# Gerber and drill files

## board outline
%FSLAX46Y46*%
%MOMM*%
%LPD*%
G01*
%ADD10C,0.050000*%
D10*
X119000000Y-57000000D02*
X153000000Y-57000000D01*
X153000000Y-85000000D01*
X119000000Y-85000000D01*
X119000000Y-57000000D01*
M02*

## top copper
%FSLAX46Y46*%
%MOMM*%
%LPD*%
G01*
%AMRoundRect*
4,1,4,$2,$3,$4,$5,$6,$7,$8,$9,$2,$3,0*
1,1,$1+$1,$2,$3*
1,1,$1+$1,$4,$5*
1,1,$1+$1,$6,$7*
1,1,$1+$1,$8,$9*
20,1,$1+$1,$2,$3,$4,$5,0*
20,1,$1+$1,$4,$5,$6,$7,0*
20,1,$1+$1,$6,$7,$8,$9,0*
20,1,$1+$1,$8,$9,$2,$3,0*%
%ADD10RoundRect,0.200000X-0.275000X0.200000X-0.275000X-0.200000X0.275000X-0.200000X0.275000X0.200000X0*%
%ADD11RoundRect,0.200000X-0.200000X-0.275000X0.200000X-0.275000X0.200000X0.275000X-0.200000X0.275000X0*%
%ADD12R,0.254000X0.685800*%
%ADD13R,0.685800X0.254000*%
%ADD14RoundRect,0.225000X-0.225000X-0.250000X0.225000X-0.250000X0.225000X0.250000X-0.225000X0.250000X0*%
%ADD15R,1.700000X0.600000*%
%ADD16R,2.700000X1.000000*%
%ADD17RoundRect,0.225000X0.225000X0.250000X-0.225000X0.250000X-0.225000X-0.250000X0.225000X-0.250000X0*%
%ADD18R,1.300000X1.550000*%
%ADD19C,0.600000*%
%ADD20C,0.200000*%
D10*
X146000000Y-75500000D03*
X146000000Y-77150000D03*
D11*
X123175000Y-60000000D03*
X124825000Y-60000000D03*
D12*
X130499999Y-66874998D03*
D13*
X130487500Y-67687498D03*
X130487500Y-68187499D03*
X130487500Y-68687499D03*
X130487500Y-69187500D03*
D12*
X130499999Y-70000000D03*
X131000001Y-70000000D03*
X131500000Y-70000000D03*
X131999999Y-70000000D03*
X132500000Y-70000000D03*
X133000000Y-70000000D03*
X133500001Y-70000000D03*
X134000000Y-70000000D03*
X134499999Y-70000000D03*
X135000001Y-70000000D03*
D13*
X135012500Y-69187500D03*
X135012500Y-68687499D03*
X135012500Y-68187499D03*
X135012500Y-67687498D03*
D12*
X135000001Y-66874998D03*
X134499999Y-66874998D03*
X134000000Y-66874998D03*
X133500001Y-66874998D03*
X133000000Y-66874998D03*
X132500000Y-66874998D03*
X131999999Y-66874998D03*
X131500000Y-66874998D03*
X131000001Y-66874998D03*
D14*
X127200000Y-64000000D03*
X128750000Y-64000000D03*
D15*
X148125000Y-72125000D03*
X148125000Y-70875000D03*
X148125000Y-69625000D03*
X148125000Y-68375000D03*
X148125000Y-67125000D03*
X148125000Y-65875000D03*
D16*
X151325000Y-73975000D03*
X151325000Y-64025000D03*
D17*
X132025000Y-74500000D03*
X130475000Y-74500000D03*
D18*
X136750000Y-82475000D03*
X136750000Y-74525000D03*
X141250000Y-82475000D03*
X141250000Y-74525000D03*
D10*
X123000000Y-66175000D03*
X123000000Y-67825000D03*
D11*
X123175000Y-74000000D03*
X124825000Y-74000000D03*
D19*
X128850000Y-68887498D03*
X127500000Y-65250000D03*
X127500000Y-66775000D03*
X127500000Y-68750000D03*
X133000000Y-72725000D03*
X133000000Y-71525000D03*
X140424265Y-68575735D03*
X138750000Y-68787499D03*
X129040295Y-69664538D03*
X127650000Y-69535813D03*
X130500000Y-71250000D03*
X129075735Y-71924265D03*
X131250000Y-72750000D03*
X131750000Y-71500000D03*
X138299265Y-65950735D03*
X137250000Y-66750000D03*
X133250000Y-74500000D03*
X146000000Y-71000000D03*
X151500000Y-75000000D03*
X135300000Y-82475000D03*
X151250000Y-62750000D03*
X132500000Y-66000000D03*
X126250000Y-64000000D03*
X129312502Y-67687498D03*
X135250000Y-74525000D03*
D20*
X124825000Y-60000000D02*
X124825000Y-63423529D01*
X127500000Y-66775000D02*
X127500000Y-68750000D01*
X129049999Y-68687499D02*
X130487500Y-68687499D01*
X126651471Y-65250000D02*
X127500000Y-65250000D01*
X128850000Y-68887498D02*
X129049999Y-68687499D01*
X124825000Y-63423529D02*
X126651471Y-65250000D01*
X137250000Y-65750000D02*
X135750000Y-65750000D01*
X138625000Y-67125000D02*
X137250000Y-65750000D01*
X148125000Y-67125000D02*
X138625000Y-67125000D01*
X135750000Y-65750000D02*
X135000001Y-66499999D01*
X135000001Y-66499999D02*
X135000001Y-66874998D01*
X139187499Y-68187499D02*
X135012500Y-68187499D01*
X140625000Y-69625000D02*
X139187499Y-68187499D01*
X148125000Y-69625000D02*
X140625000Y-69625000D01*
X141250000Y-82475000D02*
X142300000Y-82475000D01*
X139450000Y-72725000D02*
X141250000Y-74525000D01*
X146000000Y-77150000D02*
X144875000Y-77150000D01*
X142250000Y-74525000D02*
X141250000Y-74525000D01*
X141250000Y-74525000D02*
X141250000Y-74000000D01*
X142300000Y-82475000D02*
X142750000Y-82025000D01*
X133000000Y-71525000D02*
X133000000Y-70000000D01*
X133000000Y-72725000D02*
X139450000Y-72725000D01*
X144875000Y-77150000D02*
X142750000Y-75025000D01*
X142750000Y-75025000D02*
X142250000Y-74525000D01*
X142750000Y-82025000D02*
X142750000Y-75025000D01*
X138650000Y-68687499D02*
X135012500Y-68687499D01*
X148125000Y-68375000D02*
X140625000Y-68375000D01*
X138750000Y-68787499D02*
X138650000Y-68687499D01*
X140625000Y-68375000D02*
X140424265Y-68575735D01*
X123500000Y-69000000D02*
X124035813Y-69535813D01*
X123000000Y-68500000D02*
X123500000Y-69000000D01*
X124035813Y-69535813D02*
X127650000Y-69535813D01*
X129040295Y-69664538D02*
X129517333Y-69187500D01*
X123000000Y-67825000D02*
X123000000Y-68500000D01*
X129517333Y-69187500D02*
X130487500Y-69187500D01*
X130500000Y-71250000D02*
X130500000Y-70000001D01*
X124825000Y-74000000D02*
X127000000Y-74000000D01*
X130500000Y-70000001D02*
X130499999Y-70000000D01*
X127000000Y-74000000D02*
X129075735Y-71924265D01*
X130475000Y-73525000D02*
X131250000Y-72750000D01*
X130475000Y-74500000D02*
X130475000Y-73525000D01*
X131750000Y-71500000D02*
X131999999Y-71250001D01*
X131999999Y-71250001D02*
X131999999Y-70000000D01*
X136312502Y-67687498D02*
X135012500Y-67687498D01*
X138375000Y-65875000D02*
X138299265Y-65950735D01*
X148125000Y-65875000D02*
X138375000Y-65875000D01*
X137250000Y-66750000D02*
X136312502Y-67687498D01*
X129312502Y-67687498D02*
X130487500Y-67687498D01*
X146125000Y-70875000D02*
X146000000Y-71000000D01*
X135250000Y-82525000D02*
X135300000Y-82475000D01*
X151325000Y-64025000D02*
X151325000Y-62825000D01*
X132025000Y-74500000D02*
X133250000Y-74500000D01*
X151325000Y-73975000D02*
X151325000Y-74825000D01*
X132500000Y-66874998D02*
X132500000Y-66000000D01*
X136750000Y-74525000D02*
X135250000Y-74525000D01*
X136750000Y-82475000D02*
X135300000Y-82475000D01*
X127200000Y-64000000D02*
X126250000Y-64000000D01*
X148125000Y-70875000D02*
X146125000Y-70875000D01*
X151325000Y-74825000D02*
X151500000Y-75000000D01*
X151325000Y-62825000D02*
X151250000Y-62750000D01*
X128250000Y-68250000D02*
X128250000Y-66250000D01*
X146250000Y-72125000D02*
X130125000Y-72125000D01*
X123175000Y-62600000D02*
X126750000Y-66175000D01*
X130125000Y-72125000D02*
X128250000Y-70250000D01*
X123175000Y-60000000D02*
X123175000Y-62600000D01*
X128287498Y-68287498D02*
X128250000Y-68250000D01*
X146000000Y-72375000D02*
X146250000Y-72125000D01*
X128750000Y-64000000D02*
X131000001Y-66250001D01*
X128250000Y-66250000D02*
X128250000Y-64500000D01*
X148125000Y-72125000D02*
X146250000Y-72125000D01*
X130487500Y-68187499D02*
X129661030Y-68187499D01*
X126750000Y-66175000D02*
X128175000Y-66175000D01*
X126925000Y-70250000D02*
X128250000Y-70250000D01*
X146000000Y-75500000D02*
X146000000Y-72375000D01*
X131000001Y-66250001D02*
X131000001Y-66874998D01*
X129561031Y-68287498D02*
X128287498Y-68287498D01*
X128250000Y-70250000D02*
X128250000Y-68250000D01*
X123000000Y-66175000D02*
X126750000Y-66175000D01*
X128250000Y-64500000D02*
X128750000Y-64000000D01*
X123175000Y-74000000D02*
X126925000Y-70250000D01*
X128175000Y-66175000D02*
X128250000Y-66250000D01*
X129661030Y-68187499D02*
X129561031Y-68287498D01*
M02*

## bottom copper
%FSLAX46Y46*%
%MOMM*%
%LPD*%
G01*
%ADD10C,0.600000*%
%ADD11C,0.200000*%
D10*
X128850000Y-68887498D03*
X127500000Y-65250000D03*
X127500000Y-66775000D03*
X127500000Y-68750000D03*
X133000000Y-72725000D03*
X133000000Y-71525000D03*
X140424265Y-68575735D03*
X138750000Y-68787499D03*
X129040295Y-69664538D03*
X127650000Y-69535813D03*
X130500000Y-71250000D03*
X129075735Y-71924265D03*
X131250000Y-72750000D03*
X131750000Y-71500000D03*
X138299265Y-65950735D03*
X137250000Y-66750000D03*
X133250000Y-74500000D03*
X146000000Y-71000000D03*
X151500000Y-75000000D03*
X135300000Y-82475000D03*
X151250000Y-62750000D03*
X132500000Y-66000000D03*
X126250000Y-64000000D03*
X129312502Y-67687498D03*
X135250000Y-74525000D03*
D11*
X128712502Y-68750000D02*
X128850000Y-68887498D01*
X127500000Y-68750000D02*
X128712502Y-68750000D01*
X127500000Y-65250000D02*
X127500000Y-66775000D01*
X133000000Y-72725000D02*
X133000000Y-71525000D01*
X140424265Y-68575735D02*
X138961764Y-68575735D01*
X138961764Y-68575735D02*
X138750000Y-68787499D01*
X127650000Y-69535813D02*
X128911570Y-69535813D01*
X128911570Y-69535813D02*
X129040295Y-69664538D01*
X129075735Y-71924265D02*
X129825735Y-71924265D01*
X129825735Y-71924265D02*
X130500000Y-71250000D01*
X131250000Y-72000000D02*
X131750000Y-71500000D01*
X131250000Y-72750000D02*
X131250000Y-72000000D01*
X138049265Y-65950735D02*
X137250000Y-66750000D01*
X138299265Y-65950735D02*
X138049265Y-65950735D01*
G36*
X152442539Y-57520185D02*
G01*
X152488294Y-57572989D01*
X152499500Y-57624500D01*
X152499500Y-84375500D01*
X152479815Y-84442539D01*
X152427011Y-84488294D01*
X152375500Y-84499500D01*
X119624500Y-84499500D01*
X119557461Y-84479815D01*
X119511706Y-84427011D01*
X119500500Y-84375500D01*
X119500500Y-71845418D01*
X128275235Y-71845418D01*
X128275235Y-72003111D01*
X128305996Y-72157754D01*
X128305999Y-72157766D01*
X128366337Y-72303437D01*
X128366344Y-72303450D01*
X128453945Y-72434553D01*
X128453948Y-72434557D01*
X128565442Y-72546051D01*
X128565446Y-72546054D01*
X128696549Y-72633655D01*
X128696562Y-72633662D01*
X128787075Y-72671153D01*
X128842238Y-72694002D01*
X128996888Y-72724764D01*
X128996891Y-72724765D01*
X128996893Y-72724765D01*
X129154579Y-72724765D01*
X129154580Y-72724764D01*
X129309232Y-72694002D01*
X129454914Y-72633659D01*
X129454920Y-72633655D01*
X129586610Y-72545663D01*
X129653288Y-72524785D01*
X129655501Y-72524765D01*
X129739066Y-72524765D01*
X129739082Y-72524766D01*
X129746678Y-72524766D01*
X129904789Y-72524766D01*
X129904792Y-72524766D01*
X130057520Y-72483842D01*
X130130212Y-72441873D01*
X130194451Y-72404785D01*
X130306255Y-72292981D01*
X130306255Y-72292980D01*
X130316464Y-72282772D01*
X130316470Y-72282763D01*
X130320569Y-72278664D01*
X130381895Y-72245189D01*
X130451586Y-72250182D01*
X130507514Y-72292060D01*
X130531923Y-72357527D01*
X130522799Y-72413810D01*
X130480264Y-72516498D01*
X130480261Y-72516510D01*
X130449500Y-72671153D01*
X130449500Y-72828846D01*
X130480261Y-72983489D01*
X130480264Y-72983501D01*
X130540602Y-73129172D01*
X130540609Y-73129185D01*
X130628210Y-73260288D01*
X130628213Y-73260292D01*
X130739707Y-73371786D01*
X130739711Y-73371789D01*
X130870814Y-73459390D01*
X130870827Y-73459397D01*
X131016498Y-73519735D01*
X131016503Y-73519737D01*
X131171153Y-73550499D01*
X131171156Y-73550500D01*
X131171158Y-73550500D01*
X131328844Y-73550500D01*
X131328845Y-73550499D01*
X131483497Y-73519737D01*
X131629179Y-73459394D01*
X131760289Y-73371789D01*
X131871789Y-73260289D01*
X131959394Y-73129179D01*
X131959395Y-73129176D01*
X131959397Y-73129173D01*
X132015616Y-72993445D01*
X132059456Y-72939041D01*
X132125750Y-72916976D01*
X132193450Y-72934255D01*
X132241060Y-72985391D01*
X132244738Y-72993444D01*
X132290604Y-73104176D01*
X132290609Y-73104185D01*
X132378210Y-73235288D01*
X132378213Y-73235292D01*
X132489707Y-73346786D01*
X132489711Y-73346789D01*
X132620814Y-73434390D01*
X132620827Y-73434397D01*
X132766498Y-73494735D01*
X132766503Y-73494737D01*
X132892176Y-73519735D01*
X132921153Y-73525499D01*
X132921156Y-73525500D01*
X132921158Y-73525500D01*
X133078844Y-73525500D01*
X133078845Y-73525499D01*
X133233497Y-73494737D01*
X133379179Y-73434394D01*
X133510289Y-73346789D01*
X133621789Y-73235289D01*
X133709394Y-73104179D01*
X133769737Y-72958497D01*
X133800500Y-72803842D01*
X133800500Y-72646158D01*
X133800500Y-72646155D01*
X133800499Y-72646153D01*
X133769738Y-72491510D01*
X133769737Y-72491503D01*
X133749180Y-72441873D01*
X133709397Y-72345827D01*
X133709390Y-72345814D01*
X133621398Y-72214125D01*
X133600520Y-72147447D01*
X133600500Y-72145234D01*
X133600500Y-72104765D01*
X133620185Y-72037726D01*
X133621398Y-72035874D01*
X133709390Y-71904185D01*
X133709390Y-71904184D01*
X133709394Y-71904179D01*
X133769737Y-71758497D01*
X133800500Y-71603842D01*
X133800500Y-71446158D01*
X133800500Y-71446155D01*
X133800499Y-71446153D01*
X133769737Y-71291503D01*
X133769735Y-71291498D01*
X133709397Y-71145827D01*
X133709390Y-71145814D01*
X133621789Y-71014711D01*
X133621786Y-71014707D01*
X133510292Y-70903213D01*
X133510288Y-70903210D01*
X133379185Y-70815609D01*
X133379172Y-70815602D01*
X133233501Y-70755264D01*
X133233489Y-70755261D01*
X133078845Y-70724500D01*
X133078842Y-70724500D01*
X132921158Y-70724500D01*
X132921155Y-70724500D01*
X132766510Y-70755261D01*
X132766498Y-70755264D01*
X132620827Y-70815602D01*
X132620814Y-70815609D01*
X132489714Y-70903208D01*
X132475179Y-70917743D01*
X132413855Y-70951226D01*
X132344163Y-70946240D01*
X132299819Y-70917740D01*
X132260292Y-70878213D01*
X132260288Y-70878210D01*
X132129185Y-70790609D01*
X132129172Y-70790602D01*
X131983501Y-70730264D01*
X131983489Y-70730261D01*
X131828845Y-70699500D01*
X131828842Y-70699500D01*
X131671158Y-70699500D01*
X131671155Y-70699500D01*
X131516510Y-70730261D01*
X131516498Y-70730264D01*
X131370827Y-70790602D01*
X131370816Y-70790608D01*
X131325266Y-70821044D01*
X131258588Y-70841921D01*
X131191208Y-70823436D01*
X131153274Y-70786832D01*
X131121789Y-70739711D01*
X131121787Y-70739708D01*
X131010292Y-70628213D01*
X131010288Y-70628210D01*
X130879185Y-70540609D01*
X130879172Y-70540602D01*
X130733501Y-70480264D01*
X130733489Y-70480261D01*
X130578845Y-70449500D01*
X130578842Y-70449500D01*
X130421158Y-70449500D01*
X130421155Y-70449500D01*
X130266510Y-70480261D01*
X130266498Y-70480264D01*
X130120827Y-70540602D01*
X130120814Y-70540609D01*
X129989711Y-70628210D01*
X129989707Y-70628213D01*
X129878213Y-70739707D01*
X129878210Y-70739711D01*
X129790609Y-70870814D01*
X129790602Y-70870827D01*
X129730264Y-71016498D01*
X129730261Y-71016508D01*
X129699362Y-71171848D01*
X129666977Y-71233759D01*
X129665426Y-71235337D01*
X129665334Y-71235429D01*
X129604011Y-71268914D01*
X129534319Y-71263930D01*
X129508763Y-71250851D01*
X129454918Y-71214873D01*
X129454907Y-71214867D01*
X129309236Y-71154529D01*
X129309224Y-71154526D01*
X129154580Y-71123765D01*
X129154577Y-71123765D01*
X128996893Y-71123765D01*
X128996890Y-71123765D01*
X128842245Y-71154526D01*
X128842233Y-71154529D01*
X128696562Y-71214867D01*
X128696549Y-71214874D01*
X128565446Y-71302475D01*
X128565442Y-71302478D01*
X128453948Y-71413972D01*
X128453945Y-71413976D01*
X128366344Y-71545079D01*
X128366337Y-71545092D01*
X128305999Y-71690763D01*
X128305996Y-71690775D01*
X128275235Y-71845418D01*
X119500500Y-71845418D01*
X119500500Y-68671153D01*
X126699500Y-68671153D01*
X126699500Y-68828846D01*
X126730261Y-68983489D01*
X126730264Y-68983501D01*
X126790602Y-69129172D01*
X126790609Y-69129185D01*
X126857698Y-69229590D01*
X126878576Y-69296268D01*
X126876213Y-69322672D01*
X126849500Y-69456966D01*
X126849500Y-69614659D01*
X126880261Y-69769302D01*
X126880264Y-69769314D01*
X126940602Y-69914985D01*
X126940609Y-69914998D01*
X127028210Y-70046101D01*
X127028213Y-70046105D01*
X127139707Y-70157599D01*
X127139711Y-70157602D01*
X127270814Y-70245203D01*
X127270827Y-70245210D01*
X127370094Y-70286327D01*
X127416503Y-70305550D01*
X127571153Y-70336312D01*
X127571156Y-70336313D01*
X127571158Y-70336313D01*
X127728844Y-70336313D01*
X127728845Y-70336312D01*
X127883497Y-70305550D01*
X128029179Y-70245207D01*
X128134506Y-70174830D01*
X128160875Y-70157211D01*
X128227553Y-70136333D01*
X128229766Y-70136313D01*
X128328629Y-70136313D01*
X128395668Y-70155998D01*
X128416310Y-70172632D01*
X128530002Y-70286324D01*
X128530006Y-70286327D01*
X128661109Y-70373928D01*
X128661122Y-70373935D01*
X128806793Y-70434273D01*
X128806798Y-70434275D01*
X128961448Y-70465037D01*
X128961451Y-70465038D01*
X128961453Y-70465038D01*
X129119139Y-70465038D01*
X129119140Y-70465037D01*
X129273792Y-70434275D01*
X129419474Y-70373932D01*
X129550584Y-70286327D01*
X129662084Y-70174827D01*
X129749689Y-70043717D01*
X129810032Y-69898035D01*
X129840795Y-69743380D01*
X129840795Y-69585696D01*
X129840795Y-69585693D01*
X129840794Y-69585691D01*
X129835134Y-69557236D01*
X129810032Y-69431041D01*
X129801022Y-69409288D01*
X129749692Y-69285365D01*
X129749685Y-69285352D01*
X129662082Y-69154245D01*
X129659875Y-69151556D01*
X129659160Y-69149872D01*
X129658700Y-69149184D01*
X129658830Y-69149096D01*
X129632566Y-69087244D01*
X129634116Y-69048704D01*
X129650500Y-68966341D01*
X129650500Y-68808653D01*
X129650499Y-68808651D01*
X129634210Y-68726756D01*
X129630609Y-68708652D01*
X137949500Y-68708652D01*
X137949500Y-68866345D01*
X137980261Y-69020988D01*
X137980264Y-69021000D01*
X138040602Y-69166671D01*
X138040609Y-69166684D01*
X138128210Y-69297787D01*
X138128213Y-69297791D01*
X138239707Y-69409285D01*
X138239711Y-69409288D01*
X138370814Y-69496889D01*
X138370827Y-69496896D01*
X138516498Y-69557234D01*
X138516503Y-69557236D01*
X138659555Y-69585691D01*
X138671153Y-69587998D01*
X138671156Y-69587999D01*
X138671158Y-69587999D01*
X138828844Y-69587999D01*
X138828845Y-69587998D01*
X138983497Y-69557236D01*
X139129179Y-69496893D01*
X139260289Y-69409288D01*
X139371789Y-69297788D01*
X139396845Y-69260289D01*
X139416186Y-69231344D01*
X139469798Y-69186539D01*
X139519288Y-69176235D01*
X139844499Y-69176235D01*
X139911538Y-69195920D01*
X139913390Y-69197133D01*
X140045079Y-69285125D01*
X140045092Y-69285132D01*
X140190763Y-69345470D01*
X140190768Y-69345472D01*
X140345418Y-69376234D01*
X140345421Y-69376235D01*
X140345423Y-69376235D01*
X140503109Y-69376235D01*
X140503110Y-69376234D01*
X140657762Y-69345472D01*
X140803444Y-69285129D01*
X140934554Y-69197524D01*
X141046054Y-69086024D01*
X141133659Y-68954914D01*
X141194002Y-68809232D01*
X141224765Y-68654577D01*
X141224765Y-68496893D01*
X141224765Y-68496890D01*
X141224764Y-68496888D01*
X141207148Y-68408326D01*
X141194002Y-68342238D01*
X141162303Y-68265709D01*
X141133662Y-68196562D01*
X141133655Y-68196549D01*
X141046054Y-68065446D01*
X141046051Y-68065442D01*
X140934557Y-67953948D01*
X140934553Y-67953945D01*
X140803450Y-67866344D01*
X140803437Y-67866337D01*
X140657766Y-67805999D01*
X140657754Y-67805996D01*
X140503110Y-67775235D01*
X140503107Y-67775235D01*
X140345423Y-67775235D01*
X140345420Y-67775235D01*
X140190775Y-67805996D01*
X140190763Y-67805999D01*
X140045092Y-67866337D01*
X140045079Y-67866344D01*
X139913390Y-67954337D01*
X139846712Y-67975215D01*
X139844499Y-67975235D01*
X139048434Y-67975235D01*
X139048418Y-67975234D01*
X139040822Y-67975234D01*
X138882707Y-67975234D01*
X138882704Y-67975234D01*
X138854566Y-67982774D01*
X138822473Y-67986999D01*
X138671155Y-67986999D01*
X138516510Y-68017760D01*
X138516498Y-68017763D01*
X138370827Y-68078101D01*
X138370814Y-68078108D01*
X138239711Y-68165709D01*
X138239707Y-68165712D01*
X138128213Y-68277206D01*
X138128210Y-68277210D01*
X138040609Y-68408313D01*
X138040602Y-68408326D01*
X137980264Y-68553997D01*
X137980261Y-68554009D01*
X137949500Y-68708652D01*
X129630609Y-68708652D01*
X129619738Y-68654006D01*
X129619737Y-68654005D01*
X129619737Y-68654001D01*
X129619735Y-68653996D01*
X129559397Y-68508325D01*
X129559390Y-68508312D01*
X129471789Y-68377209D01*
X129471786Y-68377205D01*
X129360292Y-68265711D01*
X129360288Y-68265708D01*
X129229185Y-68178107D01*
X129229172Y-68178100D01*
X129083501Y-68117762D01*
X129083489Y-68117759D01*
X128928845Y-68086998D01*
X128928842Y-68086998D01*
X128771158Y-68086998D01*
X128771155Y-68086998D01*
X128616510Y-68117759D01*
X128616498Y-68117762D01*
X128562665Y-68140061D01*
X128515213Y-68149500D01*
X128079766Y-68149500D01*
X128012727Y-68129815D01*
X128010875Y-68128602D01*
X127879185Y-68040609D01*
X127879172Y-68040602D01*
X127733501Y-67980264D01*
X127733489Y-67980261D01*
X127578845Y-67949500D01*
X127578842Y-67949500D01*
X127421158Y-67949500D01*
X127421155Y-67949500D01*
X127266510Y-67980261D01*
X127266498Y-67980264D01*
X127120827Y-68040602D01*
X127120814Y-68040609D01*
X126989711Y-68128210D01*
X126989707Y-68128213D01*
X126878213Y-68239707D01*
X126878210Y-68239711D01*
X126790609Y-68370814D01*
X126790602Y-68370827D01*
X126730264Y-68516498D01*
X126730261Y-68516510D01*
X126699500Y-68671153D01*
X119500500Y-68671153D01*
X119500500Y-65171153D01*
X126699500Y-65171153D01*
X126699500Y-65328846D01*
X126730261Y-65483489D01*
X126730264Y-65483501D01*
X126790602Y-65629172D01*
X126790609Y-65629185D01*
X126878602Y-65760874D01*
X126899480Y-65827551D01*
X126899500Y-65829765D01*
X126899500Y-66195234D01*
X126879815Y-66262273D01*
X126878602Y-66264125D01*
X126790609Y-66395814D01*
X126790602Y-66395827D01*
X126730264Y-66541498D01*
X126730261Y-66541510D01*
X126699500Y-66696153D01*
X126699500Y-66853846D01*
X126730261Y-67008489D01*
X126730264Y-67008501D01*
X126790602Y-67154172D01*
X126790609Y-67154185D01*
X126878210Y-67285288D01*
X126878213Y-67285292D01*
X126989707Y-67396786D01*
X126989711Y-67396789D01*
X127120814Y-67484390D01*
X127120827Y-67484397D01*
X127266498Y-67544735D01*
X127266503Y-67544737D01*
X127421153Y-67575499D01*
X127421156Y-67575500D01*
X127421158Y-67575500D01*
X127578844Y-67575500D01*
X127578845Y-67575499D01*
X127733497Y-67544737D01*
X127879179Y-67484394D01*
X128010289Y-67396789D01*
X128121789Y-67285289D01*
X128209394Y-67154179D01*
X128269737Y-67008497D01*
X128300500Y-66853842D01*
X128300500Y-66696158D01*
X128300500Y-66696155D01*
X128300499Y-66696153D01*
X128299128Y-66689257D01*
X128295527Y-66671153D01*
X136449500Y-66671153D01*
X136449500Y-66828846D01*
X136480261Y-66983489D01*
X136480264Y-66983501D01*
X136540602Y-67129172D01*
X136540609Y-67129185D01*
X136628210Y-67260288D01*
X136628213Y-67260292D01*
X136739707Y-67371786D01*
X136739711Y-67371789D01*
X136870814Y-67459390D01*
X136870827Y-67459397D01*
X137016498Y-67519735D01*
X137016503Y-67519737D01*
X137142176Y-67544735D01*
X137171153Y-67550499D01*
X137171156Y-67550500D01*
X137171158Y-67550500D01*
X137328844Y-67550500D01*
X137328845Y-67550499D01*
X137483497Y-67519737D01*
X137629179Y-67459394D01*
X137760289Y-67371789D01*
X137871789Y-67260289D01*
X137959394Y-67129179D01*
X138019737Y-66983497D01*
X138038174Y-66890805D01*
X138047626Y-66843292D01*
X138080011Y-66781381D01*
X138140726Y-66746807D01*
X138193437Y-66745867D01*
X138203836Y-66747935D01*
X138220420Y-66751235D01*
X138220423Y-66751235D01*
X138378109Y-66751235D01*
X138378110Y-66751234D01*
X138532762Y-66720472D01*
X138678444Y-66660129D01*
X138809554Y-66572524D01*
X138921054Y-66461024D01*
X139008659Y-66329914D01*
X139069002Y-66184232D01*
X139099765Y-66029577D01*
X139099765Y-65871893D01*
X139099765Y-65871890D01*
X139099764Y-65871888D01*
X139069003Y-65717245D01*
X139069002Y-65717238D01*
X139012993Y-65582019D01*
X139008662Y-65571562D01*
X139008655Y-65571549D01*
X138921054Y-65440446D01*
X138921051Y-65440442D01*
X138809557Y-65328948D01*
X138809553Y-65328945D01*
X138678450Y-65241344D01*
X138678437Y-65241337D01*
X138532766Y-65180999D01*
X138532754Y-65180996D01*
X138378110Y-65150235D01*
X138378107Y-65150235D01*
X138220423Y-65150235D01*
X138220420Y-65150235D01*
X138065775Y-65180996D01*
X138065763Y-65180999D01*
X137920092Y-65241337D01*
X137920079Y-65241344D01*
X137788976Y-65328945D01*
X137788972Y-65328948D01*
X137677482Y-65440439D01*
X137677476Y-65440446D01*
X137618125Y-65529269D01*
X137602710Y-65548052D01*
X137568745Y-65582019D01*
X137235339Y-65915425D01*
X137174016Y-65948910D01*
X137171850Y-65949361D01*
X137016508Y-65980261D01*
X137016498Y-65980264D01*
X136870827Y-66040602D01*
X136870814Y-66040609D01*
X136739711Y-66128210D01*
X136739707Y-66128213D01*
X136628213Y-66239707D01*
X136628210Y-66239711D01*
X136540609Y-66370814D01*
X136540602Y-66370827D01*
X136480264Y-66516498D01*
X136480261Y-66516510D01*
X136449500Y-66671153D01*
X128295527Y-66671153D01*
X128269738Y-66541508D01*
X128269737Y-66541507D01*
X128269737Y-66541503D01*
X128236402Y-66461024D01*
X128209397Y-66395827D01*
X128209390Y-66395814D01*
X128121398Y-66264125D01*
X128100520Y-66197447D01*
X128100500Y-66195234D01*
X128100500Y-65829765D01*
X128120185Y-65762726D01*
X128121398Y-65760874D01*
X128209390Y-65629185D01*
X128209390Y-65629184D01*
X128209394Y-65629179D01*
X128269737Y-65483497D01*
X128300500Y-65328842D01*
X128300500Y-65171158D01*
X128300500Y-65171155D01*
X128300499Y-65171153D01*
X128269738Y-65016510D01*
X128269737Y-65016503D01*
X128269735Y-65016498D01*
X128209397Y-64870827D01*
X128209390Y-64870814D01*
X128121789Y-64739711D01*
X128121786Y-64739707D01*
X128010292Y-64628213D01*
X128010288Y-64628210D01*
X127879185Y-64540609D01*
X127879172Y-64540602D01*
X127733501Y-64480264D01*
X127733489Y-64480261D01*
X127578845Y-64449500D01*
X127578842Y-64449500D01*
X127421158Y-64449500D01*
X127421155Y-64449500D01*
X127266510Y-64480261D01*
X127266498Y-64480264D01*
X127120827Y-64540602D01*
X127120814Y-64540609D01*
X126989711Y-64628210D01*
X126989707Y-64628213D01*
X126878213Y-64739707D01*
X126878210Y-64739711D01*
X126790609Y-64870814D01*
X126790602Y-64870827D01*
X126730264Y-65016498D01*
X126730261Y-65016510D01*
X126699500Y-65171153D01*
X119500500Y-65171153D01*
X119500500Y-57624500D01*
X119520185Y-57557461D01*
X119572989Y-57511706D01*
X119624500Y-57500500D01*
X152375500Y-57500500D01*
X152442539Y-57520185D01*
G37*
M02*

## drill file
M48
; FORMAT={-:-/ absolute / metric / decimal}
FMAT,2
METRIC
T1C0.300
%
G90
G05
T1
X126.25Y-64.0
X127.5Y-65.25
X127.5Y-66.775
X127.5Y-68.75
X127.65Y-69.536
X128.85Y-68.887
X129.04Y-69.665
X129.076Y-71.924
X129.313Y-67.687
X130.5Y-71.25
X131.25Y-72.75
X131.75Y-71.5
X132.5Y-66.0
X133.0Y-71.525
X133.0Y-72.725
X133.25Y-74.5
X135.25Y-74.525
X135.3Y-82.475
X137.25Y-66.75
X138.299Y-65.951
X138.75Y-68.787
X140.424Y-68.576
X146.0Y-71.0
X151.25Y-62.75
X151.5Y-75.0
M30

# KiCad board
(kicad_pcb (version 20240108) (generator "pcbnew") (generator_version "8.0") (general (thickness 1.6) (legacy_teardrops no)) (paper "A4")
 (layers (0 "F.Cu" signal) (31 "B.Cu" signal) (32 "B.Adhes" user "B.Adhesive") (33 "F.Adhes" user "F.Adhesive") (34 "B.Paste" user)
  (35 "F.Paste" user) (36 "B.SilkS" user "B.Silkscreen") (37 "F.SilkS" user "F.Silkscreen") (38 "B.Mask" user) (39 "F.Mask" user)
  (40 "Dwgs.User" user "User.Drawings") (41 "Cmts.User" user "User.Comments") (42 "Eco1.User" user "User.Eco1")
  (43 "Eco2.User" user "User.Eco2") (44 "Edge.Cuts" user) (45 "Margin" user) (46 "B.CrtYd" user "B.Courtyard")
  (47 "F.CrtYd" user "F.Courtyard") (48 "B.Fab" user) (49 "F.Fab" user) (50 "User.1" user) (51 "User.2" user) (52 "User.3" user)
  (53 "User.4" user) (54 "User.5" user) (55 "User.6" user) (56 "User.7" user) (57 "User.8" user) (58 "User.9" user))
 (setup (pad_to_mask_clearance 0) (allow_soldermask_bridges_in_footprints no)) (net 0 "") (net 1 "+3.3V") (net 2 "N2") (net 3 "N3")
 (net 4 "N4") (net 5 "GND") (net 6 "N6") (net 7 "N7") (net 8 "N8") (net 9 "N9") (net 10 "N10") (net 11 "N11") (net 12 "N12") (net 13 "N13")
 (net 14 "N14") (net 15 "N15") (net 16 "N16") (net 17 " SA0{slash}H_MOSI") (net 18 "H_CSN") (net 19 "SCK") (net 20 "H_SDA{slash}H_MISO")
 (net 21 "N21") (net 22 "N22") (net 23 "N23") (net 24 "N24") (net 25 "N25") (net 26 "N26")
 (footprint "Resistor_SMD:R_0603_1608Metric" (layer "F.Cu") (at 146 76.325 -90)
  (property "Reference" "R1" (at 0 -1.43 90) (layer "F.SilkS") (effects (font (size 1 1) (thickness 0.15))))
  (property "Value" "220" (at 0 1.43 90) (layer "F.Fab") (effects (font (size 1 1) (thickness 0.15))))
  (pad "1" smd roundrect (at -0.825 0 270) (size 0.8 0.95) (layers "F.Cu" "F.Paste" "F.Mask") (roundrect_rratio 0.25) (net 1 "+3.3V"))
  (pad "2" smd roundrect (at 0.825 0 270) (size 0.8 0.95) (layers "F.Cu" "F.Paste" "F.Mask") (roundrect_rratio 0.25) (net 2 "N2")))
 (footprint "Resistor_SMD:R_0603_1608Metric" (layer "F.Cu") (at 124 60)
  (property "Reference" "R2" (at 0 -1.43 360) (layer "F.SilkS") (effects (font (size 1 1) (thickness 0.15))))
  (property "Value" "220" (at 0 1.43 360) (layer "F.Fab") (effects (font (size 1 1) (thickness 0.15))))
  (pad "1" smd roundrect (at -0.825 0) (size 0.8 0.95) (layers "F.Cu" "F.Paste" "F.Mask") (roundrect_rratio 0.25) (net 1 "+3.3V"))
  (pad "2" smd roundrect (at 0.825 0) (size 0.8 0.95) (layers "F.Cu" "F.Paste" "F.Mask") (roundrect_rratio 0.25) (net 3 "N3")))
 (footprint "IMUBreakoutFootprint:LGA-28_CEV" (layer "F.Cu") (at 132.75 68.437499 90)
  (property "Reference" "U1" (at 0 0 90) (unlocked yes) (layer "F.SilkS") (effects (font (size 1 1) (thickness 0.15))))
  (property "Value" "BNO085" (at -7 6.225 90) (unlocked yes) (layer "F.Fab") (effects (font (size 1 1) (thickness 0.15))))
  (pad "1" smd rect (at 1.562501 -2.250001 90) (size 0.6858 0.254) (layers "F.Cu" "F.Paste" "F.Mask") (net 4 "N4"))
  (pad "2" smd rect (at 0.750001 -2.2625 180) (size 0.6858 0.254) (layers "F.Cu" "F.Paste" "F.Mask") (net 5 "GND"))
  (pad "3" smd rect (at 0.25 -2.2625 180) (size 0.6858 0.254) (layers "F.Cu" "F.Paste" "F.Mask") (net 1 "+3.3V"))
  (pad "4" smd rect (at -0.25 -2.2625 180) (size 0.6858 0.254) (layers "F.Cu" "F.Paste" "F.Mask") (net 3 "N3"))
  (pad "5" smd rect (at -0.750001 -2.2625 180) (size 0.6858 0.254) (layers "F.Cu" "F.Paste" "F.Mask") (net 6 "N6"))
  (pad "6" smd rect (at -1.562501 -2.250001 90) (size 0.6858 0.254) (layers "F.Cu" "F.Paste" "F.Mask") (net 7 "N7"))
  (pad "7" smd rect (at -1.562501 -1.749999 90) (size 0.6858 0.254) (layers "F.Cu" "F.Paste" "F.Mask") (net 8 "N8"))
  (pad "8" smd rect (at -1.562501 -1.25 90) (size 0.6858 0.254) (layers "F.Cu" "F.Paste" "F.Mask") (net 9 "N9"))
  (pad "9" smd rect (at -1.562501 -0.750001 90) (size 0.6858 0.254) (layers "F.Cu" "F.Paste" "F.Mask") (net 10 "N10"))
  (pad "10" smd rect (at -1.562501 -0.25 90) (size 0.6858 0.254) (layers "F.Cu" "F.Paste" "F.Mask") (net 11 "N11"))
  (pad "11" smd rect (at -1.562501 0.25 90) (size 0.6858 0.254) (layers "F.Cu" "F.Paste" "F.Mask") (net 2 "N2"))
  (pad "12" smd rect (at -1.562501 0.750001 90) (size 0.6858 0.254) (layers "F.Cu" "F.Paste" "F.Mask") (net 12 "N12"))
  (pad "13" smd rect (at -1.562501 1.25 90) (size 0.6858 0.254) (layers "F.Cu" "F.Paste" "F.Mask") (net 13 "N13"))
  (pad "14" smd rect (at -1.562501 1.749999 90) (size 0.6858 0.254) (layers "F.Cu" "F.Paste" "F.Mask") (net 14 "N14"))
  (pad "15" smd rect (at -1.562501 2.250001 90) (size 0.6858 0.254) (layers "F.Cu" "F.Paste" "F.Mask") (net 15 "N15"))
  (pad "16" smd rect (at -0.750001 2.2625 180) (size 0.6858 0.254) (layers "F.Cu" "F.Paste" "F.Mask") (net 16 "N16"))
  (pad "17" smd rect (at -0.25 2.2625 180) (size 0.6858 0.254) (layers "F.Cu" "F.Paste" "F.Mask") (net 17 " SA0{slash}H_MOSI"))
  (pad "18" smd rect (at 0.25 2.2625 180) (size 0.6858 0.254) (layers "F.Cu" "F.Paste" "F.Mask") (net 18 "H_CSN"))
  (pad "19" smd rect (at 0.750001 2.2625 180) (size 0.6858 0.254) (layers "F.Cu" "F.Paste" "F.Mask") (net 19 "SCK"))
  (pad "20" smd rect (at 1.562501 2.250001 90) (size 0.6858 0.254) (layers "F.Cu" "F.Paste" "F.Mask") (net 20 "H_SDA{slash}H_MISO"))
  (pad "21" smd rect (at 1.562501 1.749999 90) (size 0.6858 0.254) (layers "F.Cu" "F.Paste" "F.Mask") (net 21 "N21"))
  (pad "22" smd rect (at 1.562501 1.25 90) (size 0.6858 0.254) (layers "F.Cu" "F.Paste" "F.Mask") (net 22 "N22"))
  (pad "23" smd rect (at 1.562501 0.750001 90) (size 0.6858 0.254) (layers "F.Cu" "F.Paste" "F.Mask") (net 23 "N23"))
  (pad "24" smd rect (at 1.562501 0.25 90) (size 0.6858 0.254) (layers "F.Cu" "F.Paste" "F.Mask") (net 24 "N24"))
  (pad "25" smd rect (at 1.562501 -0.25 90) (size 0.6858 0.254) (layers "F.Cu" "F.Paste" "F.Mask") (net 5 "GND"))
  (pad "26" smd rect (at 1.562501 -0.750001 90) (size 0.6858 0.254) (layers "F.Cu" "F.Paste" "F.Mask") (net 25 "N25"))
  (pad "27" smd rect (at 1.562501 -1.25 90) (size 0.6858 0.254) (layers "F.Cu" "F.Paste" "F.Mask") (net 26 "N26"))
  (pad "28" smd rect (at 1.562501 -1.749999 90) (size 0.6858 0.254) (layers "F.Cu" "F.Paste" "F.Mask") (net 1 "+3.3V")))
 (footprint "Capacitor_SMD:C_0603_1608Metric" (layer "F.Cu") (at 127.975 64)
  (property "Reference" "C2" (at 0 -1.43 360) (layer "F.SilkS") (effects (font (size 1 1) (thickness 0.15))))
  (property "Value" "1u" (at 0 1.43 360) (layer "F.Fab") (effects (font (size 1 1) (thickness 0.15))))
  (pad "1" smd roundrect (at -0.775 0) (size 0.9 0.95) (layers "F.Cu" "F.Paste" "F.Mask") (roundrect_rratio 0.25) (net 5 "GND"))
  (pad "2" smd roundrect (at 0.775 0) (size 0.9 0.95) (layers "F.Cu" "F.Paste" "F.Mask") (roundrect_rratio 0.25) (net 1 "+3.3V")))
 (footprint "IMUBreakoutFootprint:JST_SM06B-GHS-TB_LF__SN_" (layer "F.Cu") (at 150 69 90)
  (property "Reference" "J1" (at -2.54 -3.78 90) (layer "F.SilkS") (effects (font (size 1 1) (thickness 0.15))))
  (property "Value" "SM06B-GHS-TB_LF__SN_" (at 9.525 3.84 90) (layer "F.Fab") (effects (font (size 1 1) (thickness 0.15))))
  (pad "1" smd rect (at -3.125 -1.875 90) (size 0.6 1.7) (layers "F.Cu" "F.Paste" "F.Mask") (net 1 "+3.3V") (solder_mask_margin 0.102))
  (pad "2" smd rect (at -1.875 -1.875 90) (size 0.6 1.7) (layers "F.Cu" "F.Paste" "F.Mask") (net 5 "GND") (solder_mask_margin 0.102))
  (pad "3" smd rect (at -0.625 -1.875 90) (size 0.6 1.7) (layers "F.Cu" "F.Paste" "F.Mask") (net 18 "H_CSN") (solder_mask_margin 0.102))
  (pad "4" smd rect (at 0.625 -1.875 90) (size 0.6 1.7) (layers "F.Cu" "F.Paste" "F.Mask") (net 17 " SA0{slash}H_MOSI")
   (solder_mask_margin 0.102))
  (pad "5" smd rect (at 1.875 -1.875 90) (size 0.6 1.7) (layers "F.Cu" "F.Paste" "F.Mask") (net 20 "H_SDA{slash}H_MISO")
   (solder_mask_margin 0.102))
  (pad "6" smd rect (at 3.125 -1.875 90) (size 0.6 1.7) (layers "F.Cu" "F.Paste" "F.Mask") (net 19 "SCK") (solder_mask_margin 0.102))
  (pad "S1" smd rect (at -4.975 1.325 90) (size 1 2.7) (layers "F.Cu" "F.Paste" "F.Mask") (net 5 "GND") (solder_mask_margin 0.102))
  (pad "S2" smd rect (at 4.975 1.325 90) (size 1 2.7) (layers "F.Cu" "F.Paste" "F.Mask") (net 5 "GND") (solder_mask_margin 0.102)))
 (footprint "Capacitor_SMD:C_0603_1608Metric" (layer "F.Cu") (at 131.25 74.5 180)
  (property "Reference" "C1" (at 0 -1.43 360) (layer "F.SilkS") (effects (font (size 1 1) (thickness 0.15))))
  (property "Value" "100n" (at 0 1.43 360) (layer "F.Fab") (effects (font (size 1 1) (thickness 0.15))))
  (pad "1" smd roundrect (at -0.775 0 180) (size 0.9 0.95) (layers "F.Cu" "F.Paste" "F.Mask") (roundrect_rratio 0.25) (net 5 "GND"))
  (pad "2" smd roundrect (at 0.775 0 180) (size 0.9 0.95) (layers "F.Cu" "F.Paste" "F.Mask") (roundrect_rratio 0.25) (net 10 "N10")))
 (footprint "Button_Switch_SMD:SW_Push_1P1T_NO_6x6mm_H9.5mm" (layer "F.Cu") (at 139 78.5 90)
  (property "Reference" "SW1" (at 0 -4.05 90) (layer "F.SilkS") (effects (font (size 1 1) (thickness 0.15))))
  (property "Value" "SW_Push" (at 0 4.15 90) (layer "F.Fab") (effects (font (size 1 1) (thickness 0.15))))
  (pad "1" smd rect (at -3.975 -2.25 90) (size 1.55 1.3) (layers "F.Cu" "F.Paste" "F.Mask") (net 5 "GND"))
  (pad "1" smd rect (at 3.975 -2.25 90) (size 1.55 1.3) (layers "F.Cu" "F.Paste" "F.Mask") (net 5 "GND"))
  (pad "2" smd rect (at -3.975 2.25 90) (size 1.55 1.3) (layers "F.Cu" "F.Paste" "F.Mask") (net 2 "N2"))
  (pad "2" smd rect (at 3.975 2.25 90) (size 1.55 1.3) (layers "F.Cu" "F.Paste" "F.Mask") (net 2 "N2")))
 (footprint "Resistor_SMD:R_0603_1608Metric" (layer "F.Cu") (at 123 67 -90)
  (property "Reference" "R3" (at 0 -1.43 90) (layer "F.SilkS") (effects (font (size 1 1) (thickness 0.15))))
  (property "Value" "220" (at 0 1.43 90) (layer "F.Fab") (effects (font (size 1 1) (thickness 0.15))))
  (pad "1" smd roundrect (at -0.825 0 270) (size 0.8 0.95) (layers "F.Cu" "F.Paste" "F.Mask") (roundrect_rratio 0.25) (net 1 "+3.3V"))
  (pad "2" smd roundrect (at 0.825 0 270) (size 0.8 0.95) (layers "F.Cu" "F.Paste" "F.Mask") (roundrect_rratio 0.25) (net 6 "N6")))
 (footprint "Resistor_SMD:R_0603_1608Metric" (layer "F.Cu") (at 124 74)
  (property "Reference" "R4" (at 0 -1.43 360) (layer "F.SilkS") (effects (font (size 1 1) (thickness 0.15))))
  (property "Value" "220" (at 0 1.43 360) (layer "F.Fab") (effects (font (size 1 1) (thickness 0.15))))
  (pad "1" smd roundrect (at -0.825 0) (size 0.8 0.95) (layers "F.Cu" "F.Paste" "F.Mask") (roundrect_rratio 0.25) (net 1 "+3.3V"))
  (pad "2" smd roundrect (at 0.825 0) (size 0.8 0.95) (layers "F.Cu" "F.Paste" "F.Mask") (roundrect_rratio 0.25) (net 7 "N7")))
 (gr_rect (start 119 57) (end 153 85) (stroke (width 0.05) (type default)) (fill none) (layer "Edge.Cuts"))
 (segment (start 124.825 60) (end 124.825 63.423529) (width 0.2) (layer "F.Cu") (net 3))
 (segment (start 127.5 66.775) (end 127.5 68.75) (width 0.2) (layer "F.Cu") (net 3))
 (segment (start 129.049999 68.687499) (end 130.4875 68.687499) (width 0.2) (layer "F.Cu") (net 3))
 (segment (start 126.651471 65.25) (end 127.5 65.25) (width 0.2) (layer "F.Cu") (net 3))
 (segment (start 128.85 68.887498) (end 129.049999 68.687499) (width 0.2) (layer "F.Cu") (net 3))
 (segment (start 124.825 63.423529) (end 126.651471 65.25) (width 0.2) (layer "F.Cu") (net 3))
 (via (at 128.85 68.887498) (size 0.6) (drill 0.3) (layers "F.Cu" "B.Cu") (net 3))
 (via (at 127.5 65.25) (size 0.6) (drill 0.3) (layers "F.Cu" "B.Cu") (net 3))
 (via (at 127.5 66.775) (size 0.6) (drill 0.3) (layers "F.Cu" "B.Cu") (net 3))
 (via (at 127.5 68.75) (size 0.6) (drill 0.3) (layers "F.Cu" "B.Cu") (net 3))
 (segment (start 128.712502 68.75) (end 128.85 68.887498) (width 0.2) (layer "B.Cu") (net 3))
 (segment (start 127.5 68.75) (end 128.712502 68.75) (width 0.2) (layer "B.Cu") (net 3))
 (segment (start 127.5 65.25) (end 127.5 66.775) (width 0.2) (layer "B.Cu") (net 3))
 (segment (start 137.25 65.75) (end 135.75 65.75) (width 0.2) (layer "F.Cu") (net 20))
 (segment (start 138.625 67.125) (end 137.25 65.75) (width 0.2) (layer "F.Cu") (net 20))
 (segment (start 148.125 67.125) (end 138.625 67.125) (width 0.2) (layer "F.Cu") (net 20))
 (segment (start 135.75 65.75) (end 135.000001 66.499999) (width 0.2) (layer "F.Cu") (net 20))
 (segment (start 135.000001 66.499999) (end 135.000001 66.874998) (width 0.2) (layer "F.Cu") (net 20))
 (segment (start 139.187499 68.187499) (end 135.0125 68.187499) (width 0.2) (layer "F.Cu") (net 18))
 (segment (start 140.625 69.625) (end 139.187499 68.187499) (width 0.2) (layer "F.Cu") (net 18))
 (segment (start 148.125 69.625) (end 140.625 69.625) (width 0.2) (layer "F.Cu") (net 18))
 (segment (start 141.25 82.475) (end 142.3 82.475) (width 0.2) (layer "F.Cu") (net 2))
 (segment (start 139.45 72.725) (end 141.25 74.525) (width 0.2) (layer "F.Cu") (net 2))
 (segment (start 146 77.15) (end 144.875 77.15) (width 0.2) (layer "F.Cu") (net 2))
 (segment (start 142.25 74.525) (end 141.25 74.525) (width 0.2) (layer "F.Cu") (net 2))
 (segment (start 141.25 74.525) (end 141.25 74) (width 0.2) (layer "F.Cu") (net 2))
 (segment (start 142.3 82.475) (end 142.75 82.025) (width 0.2) (layer "F.Cu") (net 2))
 (segment (start 133 71.525) (end 133 70) (width 0.2) (layer "F.Cu") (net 2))
 (segment (start 133 72.725) (end 139.45 72.725) (width 0.2) (layer "F.Cu") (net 2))
 (segment (start 144.875 77.15) (end 142.75 75.025) (width 0.2) (layer "F.Cu") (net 2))
 (segment (start 142.75 75.025) (end 142.25 74.525) (width 0.2) (layer "F.Cu") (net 2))
 (segment (start 142.75 82.025) (end 142.75 75.025) (width 0.2) (layer "F.Cu") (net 2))
 (via (at 133 72.725) (size 0.6) (drill 0.3) (layers "F.Cu" "B.Cu") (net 2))
 (via (at 133 71.525) (size 0.6) (drill 0.3) (layers "F.Cu" "B.Cu") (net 2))
 (segment (start 133 72.725) (end 133 71.525) (width 0.2) (layer "B.Cu") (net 2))
 (segment (start 138.65 68.687499) (end 135.0125 68.687499) (width 0.2) (layer "F.Cu") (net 17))
 (segment (start 148.125 68.375) (end 140.625 68.375) (width 0.2) (layer "F.Cu") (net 17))
 (segment (start 138.75 68.787499) (end 138.65 68.687499) (width 0.2) (layer "F.Cu") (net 17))
 (segment (start 140.625 68.375) (end 140.424265 68.575735) (width 0.2) (layer "F.Cu") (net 17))
 (via (at 140.424265 68.575735) (size 0.6) (drill 0.3) (layers "F.Cu" "B.Cu") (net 17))
 (via (at 138.75 68.787499) (size 0.6) (drill 0.3) (layers "F.Cu" "B.Cu") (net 17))
 (segment (start 140.424265 68.575735) (end 138.961764 68.575735) (width 0.2) (layer "B.Cu") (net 17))
 (segment (start 138.961764 68.575735) (end 138.75 68.787499) (width 0.2) (layer "B.Cu") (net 17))
 (segment (start 123.5 69) (end 124.035813 69.535813) (width 0.2) (layer "F.Cu") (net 6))
 (segment (start 123 68.5) (end 123.5 69) (width 0.2) (layer "F.Cu") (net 6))
 (segment (start 124.035813 69.535813) (end 127.65 69.535813) (width 0.2) (layer "F.Cu") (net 6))
 (segment (start 129.040295 69.664538) (end 129.517333 69.1875) (width 0.2) (layer "F.Cu") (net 6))
 (segment (start 123 67.825) (end 123 68.5) (width 0.2) (layer "F.Cu") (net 6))
 (segment (start 129.517333 69.1875) (end 130.4875 69.1875) (width 0.2) (layer "F.Cu") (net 6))
 (via (at 129.040295 69.664538) (size 0.6) (drill 0.3) (layers "F.Cu" "B.Cu") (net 6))
 (via (at 127.65 69.535813) (size 0.6) (drill 0.3) (layers "F.Cu" "B.Cu") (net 6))
 (segment (start 127.65 69.535813) (end 128.91157 69.535813) (width 0.2) (layer "B.Cu") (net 6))
 (segment (start 128.91157 69.535813) (end 129.040295 69.664538) (width 0.2) (layer "B.Cu") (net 6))
 (segment (start 130.5 71.25) (end 130.5 70.000001) (width 0.2) (layer "F.Cu") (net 7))
 (segment (start 124.825 74) (end 127 74) (width 0.2) (layer "F.Cu") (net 7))
 (segment (start 130.5 70.000001) (end 130.499999 70) (width 0.2) (layer "F.Cu") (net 7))
 (segment (start 127 74) (end 129.075735 71.924265) (width 0.2) (layer "F.Cu") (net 7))
 (via (at 130.5 71.25) (size 0.6) (drill 0.3) (layers "F.Cu" "B.Cu") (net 7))
 (via (at 129.075735 71.924265) (size 0.6) (drill 0.3) (layers "F.Cu" "B.Cu") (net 7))
 (segment (start 129.075735 71.924265) (end 129.825735 71.924265) (width 0.2) (layer "B.Cu") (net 7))
 (segment (start 129.825735 71.924265) (end 130.5 71.25) (width 0.2) (layer "B.Cu") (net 7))
 (segment (start 130.475 73.525) (end 131.25 72.75) (width 0.2) (layer "F.Cu") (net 10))
 (segment (start 130.475 74.5) (end 130.475 73.525) (width 0.2) (layer "F.Cu") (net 10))
 (segment (start 131.75 71.5) (end 131.999999 71.250001) (width 0.2) (layer "F.Cu") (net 10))
 (segment (start 131.999999 71.250001) (end 131.999999 70) (width 0.2) (layer "F.Cu") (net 10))
 (via (at 131.25 72.75) (size 0.6) (drill 0.3) (layers "F.Cu" "B.Cu") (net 10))
 (via (at 131.75 71.5) (size 0.6) (drill 0.3) (layers "F.Cu" "B.Cu") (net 10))
 (segment (start 131.25 72) (end 131.75 71.5) (width 0.2) (layer "B.Cu") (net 10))
 (segment (start 131.25 72.75) (end 131.25 72) (width 0.2) (layer "B.Cu") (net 10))
 (segment (start 136.312502 67.687498) (end 135.0125 67.687498) (width 0.2) (layer "F.Cu") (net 19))
 (segment (start 138.375 65.875) (end 138.299265 65.950735) (width 0.2) (layer "F.Cu") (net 19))
 (segment (start 148.125 65.875) (end 138.375 65.875) (width 0.2) (layer "F.Cu") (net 19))
 (segment (start 137.25 66.75) (end 136.312502 67.687498) (width 0.2) (layer "F.Cu") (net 19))
 (via (at 138.299265 65.950735) (size 0.6) (drill 0.3) (layers "F.Cu" "B.Cu") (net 19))
 (via (at 137.25 66.75) (size 0.6) (drill 0.3) (layers "F.Cu" "B.Cu") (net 19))
 (segment (start 138.049265 65.950735) (end 137.25 66.75) (width 0.2) (layer "B.Cu") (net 19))
 (segment (start 138.299265 65.950735) (end 138.049265 65.950735) (width 0.2) (layer "B.Cu") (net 19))
 (segment (start 129.312502 67.687498) (end 130.4875 67.687498) (width 0.2) (layer "F.Cu") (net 5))
 (segment (start 146.125 70.875) (end 146 71) (width 0.2) (layer "F.Cu") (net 5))
 (segment (start 135.25 82.525) (end 135.3 82.475) (width 0.2) (layer "F.Cu") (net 5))
 (segment (start 151.325 64.025) (end 151.325 62.825) (width 0.2) (layer "F.Cu") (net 5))
 (segment (start 132.025 74.5) (end 133.25 74.5) (width 0.2) (layer "F.Cu") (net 5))
 (segment (start 151.325 73.975) (end 151.325 74.825) (width 0.2) (layer "F.Cu") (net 5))
 (segment (start 132.5 66.874998) (end 132.5 66) (width 0.2) (layer "F.Cu") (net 5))
 (segment (start 136.75 74.525) (end 135.25 74.525) (width 0.2) (layer "F.Cu") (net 5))
 (segment (start 136.75 82.475) (end 135.3 82.475) (width 0.2) (layer "F.Cu") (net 5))
 (segment (start 127.2 64) (end 126.25 64) (width 0.2) (layer "F.Cu") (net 5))
 (segment (start 148.125 70.875) (end 146.125 70.875) (width 0.2) (layer "F.Cu") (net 5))
 (segment (start 151.325 74.825) (end 151.5 75) (width 0.2) (layer "F.Cu") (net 5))
 (segment (start 151.325 62.825) (end 151.25 62.75) (width 0.2) (layer "F.Cu") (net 5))
 (via (at 133.25 74.5) (size 0.6) (drill 0.3) (layers "F.Cu" "B.Cu") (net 5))
 (via (at 146 71) (size 0.6) (drill 0.3) (layers "F.Cu" "B.Cu") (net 5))
 (via (at 151.5 75) (size 0.6) (drill 0.3) (layers "F.Cu" "B.Cu") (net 5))
 (via (at 135.3 82.475) (size 0.6) (drill 0.3) (layers "F.Cu" "B.Cu") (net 5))
 (via (at 151.25 62.75) (size 0.6) (drill 0.3) (layers "F.Cu" "B.Cu") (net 5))
 (via (at 132.5 66) (size 0.6) (drill 0.3) (layers "F.Cu" "B.Cu") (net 5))
 (via (at 126.25 64) (size 0.6) (drill 0.3) (layers "F.Cu" "B.Cu") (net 5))
 (via (at 129.312502 67.687498) (size 0.6) (drill 0.3) (layers "F.Cu" "B.Cu") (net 5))
 (via (at 135.25 74.525) (size 0.6) (drill 0.3) (layers "F.Cu" "B.Cu") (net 5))
 (segment (start 128.25 68.25) (end 128.25 66.25) (width 0.2) (layer "F.Cu") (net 1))
 (segment (start 146.25 72.125) (end 130.125 72.125) (width 0.2) (layer "F.Cu") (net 1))
 (segment (start 123.175 62.6) (end 126.75 66.175) (width 0.2) (layer "F.Cu") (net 1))
 (segment (start 130.125 72.125) (end 128.25 70.25) (width 0.2) (layer "F.Cu") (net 1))
 (segment (start 123.175 60) (end 123.175 62.6) (width 0.2) (layer "F.Cu") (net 1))
 (segment (start 128.287498 68.287498) (end 128.25 68.25) (width 0.2) (layer "F.Cu") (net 1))
 (segment (start 146 72.375) (end 146.25 72.125) (width 0.2) (layer "F.Cu") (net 1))
 (segment (start 128.75 64) (end 131.000001 66.250001) (width 0.2) (layer "F.Cu") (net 1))
 (segment (start 128.25 66.25) (end 128.25 64.5) (width 0.2) (layer "F.Cu") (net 1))
 (segment (start 148.125 72.125) (end 146.25 72.125) (width 0.2) (layer "F.Cu") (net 1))
 (segment (start 130.4875 68.187499) (end 129.66103 68.187499) (width 0.2) (layer "F.Cu") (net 1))
 (segment (start 126.75 66.175) (end 128.175 66.175) (width 0.2) (layer "F.Cu") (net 1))
 (segment (start 126.925 70.25) (end 128.25 70.25) (width 0.2) (layer "F.Cu") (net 1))
 (segment (start 146 75.5) (end 146 72.375) (width 0.2) (layer "F.Cu") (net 1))
 (segment (start 131.000001 66.250001) (end 131.000001 66.874998) (width 0.2) (layer "F.Cu") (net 1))
 (segment (start 129.561031 68.287498) (end 128.287498 68.287498) (width 0.2) (layer "F.Cu") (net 1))
 (segment (start 128.25 70.25) (end 128.25 68.25) (width 0.2) (layer "F.Cu") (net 1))
 (segment (start 123 66.175) (end 126.75 66.175) (width 0.2) (layer "F.Cu") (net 1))
 (segment (start 128.25 64.5) (end 128.75 64) (width 0.2) (layer "F.Cu") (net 1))
 (segment (start 123.175 74) (end 126.925 70.25) (width 0.2) (layer "F.Cu") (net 1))
 (segment (start 128.175 66.175) (end 128.25 66.25) (width 0.2) (layer "F.Cu") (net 1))
 (segment (start 129.66103 68.187499) (end 129.561031 68.287498) (width 0.2) (layer "F.Cu") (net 1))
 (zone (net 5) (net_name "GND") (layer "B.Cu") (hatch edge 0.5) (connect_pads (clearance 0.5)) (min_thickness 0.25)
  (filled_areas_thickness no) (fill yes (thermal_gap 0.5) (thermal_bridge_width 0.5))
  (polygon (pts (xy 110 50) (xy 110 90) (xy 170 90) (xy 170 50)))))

